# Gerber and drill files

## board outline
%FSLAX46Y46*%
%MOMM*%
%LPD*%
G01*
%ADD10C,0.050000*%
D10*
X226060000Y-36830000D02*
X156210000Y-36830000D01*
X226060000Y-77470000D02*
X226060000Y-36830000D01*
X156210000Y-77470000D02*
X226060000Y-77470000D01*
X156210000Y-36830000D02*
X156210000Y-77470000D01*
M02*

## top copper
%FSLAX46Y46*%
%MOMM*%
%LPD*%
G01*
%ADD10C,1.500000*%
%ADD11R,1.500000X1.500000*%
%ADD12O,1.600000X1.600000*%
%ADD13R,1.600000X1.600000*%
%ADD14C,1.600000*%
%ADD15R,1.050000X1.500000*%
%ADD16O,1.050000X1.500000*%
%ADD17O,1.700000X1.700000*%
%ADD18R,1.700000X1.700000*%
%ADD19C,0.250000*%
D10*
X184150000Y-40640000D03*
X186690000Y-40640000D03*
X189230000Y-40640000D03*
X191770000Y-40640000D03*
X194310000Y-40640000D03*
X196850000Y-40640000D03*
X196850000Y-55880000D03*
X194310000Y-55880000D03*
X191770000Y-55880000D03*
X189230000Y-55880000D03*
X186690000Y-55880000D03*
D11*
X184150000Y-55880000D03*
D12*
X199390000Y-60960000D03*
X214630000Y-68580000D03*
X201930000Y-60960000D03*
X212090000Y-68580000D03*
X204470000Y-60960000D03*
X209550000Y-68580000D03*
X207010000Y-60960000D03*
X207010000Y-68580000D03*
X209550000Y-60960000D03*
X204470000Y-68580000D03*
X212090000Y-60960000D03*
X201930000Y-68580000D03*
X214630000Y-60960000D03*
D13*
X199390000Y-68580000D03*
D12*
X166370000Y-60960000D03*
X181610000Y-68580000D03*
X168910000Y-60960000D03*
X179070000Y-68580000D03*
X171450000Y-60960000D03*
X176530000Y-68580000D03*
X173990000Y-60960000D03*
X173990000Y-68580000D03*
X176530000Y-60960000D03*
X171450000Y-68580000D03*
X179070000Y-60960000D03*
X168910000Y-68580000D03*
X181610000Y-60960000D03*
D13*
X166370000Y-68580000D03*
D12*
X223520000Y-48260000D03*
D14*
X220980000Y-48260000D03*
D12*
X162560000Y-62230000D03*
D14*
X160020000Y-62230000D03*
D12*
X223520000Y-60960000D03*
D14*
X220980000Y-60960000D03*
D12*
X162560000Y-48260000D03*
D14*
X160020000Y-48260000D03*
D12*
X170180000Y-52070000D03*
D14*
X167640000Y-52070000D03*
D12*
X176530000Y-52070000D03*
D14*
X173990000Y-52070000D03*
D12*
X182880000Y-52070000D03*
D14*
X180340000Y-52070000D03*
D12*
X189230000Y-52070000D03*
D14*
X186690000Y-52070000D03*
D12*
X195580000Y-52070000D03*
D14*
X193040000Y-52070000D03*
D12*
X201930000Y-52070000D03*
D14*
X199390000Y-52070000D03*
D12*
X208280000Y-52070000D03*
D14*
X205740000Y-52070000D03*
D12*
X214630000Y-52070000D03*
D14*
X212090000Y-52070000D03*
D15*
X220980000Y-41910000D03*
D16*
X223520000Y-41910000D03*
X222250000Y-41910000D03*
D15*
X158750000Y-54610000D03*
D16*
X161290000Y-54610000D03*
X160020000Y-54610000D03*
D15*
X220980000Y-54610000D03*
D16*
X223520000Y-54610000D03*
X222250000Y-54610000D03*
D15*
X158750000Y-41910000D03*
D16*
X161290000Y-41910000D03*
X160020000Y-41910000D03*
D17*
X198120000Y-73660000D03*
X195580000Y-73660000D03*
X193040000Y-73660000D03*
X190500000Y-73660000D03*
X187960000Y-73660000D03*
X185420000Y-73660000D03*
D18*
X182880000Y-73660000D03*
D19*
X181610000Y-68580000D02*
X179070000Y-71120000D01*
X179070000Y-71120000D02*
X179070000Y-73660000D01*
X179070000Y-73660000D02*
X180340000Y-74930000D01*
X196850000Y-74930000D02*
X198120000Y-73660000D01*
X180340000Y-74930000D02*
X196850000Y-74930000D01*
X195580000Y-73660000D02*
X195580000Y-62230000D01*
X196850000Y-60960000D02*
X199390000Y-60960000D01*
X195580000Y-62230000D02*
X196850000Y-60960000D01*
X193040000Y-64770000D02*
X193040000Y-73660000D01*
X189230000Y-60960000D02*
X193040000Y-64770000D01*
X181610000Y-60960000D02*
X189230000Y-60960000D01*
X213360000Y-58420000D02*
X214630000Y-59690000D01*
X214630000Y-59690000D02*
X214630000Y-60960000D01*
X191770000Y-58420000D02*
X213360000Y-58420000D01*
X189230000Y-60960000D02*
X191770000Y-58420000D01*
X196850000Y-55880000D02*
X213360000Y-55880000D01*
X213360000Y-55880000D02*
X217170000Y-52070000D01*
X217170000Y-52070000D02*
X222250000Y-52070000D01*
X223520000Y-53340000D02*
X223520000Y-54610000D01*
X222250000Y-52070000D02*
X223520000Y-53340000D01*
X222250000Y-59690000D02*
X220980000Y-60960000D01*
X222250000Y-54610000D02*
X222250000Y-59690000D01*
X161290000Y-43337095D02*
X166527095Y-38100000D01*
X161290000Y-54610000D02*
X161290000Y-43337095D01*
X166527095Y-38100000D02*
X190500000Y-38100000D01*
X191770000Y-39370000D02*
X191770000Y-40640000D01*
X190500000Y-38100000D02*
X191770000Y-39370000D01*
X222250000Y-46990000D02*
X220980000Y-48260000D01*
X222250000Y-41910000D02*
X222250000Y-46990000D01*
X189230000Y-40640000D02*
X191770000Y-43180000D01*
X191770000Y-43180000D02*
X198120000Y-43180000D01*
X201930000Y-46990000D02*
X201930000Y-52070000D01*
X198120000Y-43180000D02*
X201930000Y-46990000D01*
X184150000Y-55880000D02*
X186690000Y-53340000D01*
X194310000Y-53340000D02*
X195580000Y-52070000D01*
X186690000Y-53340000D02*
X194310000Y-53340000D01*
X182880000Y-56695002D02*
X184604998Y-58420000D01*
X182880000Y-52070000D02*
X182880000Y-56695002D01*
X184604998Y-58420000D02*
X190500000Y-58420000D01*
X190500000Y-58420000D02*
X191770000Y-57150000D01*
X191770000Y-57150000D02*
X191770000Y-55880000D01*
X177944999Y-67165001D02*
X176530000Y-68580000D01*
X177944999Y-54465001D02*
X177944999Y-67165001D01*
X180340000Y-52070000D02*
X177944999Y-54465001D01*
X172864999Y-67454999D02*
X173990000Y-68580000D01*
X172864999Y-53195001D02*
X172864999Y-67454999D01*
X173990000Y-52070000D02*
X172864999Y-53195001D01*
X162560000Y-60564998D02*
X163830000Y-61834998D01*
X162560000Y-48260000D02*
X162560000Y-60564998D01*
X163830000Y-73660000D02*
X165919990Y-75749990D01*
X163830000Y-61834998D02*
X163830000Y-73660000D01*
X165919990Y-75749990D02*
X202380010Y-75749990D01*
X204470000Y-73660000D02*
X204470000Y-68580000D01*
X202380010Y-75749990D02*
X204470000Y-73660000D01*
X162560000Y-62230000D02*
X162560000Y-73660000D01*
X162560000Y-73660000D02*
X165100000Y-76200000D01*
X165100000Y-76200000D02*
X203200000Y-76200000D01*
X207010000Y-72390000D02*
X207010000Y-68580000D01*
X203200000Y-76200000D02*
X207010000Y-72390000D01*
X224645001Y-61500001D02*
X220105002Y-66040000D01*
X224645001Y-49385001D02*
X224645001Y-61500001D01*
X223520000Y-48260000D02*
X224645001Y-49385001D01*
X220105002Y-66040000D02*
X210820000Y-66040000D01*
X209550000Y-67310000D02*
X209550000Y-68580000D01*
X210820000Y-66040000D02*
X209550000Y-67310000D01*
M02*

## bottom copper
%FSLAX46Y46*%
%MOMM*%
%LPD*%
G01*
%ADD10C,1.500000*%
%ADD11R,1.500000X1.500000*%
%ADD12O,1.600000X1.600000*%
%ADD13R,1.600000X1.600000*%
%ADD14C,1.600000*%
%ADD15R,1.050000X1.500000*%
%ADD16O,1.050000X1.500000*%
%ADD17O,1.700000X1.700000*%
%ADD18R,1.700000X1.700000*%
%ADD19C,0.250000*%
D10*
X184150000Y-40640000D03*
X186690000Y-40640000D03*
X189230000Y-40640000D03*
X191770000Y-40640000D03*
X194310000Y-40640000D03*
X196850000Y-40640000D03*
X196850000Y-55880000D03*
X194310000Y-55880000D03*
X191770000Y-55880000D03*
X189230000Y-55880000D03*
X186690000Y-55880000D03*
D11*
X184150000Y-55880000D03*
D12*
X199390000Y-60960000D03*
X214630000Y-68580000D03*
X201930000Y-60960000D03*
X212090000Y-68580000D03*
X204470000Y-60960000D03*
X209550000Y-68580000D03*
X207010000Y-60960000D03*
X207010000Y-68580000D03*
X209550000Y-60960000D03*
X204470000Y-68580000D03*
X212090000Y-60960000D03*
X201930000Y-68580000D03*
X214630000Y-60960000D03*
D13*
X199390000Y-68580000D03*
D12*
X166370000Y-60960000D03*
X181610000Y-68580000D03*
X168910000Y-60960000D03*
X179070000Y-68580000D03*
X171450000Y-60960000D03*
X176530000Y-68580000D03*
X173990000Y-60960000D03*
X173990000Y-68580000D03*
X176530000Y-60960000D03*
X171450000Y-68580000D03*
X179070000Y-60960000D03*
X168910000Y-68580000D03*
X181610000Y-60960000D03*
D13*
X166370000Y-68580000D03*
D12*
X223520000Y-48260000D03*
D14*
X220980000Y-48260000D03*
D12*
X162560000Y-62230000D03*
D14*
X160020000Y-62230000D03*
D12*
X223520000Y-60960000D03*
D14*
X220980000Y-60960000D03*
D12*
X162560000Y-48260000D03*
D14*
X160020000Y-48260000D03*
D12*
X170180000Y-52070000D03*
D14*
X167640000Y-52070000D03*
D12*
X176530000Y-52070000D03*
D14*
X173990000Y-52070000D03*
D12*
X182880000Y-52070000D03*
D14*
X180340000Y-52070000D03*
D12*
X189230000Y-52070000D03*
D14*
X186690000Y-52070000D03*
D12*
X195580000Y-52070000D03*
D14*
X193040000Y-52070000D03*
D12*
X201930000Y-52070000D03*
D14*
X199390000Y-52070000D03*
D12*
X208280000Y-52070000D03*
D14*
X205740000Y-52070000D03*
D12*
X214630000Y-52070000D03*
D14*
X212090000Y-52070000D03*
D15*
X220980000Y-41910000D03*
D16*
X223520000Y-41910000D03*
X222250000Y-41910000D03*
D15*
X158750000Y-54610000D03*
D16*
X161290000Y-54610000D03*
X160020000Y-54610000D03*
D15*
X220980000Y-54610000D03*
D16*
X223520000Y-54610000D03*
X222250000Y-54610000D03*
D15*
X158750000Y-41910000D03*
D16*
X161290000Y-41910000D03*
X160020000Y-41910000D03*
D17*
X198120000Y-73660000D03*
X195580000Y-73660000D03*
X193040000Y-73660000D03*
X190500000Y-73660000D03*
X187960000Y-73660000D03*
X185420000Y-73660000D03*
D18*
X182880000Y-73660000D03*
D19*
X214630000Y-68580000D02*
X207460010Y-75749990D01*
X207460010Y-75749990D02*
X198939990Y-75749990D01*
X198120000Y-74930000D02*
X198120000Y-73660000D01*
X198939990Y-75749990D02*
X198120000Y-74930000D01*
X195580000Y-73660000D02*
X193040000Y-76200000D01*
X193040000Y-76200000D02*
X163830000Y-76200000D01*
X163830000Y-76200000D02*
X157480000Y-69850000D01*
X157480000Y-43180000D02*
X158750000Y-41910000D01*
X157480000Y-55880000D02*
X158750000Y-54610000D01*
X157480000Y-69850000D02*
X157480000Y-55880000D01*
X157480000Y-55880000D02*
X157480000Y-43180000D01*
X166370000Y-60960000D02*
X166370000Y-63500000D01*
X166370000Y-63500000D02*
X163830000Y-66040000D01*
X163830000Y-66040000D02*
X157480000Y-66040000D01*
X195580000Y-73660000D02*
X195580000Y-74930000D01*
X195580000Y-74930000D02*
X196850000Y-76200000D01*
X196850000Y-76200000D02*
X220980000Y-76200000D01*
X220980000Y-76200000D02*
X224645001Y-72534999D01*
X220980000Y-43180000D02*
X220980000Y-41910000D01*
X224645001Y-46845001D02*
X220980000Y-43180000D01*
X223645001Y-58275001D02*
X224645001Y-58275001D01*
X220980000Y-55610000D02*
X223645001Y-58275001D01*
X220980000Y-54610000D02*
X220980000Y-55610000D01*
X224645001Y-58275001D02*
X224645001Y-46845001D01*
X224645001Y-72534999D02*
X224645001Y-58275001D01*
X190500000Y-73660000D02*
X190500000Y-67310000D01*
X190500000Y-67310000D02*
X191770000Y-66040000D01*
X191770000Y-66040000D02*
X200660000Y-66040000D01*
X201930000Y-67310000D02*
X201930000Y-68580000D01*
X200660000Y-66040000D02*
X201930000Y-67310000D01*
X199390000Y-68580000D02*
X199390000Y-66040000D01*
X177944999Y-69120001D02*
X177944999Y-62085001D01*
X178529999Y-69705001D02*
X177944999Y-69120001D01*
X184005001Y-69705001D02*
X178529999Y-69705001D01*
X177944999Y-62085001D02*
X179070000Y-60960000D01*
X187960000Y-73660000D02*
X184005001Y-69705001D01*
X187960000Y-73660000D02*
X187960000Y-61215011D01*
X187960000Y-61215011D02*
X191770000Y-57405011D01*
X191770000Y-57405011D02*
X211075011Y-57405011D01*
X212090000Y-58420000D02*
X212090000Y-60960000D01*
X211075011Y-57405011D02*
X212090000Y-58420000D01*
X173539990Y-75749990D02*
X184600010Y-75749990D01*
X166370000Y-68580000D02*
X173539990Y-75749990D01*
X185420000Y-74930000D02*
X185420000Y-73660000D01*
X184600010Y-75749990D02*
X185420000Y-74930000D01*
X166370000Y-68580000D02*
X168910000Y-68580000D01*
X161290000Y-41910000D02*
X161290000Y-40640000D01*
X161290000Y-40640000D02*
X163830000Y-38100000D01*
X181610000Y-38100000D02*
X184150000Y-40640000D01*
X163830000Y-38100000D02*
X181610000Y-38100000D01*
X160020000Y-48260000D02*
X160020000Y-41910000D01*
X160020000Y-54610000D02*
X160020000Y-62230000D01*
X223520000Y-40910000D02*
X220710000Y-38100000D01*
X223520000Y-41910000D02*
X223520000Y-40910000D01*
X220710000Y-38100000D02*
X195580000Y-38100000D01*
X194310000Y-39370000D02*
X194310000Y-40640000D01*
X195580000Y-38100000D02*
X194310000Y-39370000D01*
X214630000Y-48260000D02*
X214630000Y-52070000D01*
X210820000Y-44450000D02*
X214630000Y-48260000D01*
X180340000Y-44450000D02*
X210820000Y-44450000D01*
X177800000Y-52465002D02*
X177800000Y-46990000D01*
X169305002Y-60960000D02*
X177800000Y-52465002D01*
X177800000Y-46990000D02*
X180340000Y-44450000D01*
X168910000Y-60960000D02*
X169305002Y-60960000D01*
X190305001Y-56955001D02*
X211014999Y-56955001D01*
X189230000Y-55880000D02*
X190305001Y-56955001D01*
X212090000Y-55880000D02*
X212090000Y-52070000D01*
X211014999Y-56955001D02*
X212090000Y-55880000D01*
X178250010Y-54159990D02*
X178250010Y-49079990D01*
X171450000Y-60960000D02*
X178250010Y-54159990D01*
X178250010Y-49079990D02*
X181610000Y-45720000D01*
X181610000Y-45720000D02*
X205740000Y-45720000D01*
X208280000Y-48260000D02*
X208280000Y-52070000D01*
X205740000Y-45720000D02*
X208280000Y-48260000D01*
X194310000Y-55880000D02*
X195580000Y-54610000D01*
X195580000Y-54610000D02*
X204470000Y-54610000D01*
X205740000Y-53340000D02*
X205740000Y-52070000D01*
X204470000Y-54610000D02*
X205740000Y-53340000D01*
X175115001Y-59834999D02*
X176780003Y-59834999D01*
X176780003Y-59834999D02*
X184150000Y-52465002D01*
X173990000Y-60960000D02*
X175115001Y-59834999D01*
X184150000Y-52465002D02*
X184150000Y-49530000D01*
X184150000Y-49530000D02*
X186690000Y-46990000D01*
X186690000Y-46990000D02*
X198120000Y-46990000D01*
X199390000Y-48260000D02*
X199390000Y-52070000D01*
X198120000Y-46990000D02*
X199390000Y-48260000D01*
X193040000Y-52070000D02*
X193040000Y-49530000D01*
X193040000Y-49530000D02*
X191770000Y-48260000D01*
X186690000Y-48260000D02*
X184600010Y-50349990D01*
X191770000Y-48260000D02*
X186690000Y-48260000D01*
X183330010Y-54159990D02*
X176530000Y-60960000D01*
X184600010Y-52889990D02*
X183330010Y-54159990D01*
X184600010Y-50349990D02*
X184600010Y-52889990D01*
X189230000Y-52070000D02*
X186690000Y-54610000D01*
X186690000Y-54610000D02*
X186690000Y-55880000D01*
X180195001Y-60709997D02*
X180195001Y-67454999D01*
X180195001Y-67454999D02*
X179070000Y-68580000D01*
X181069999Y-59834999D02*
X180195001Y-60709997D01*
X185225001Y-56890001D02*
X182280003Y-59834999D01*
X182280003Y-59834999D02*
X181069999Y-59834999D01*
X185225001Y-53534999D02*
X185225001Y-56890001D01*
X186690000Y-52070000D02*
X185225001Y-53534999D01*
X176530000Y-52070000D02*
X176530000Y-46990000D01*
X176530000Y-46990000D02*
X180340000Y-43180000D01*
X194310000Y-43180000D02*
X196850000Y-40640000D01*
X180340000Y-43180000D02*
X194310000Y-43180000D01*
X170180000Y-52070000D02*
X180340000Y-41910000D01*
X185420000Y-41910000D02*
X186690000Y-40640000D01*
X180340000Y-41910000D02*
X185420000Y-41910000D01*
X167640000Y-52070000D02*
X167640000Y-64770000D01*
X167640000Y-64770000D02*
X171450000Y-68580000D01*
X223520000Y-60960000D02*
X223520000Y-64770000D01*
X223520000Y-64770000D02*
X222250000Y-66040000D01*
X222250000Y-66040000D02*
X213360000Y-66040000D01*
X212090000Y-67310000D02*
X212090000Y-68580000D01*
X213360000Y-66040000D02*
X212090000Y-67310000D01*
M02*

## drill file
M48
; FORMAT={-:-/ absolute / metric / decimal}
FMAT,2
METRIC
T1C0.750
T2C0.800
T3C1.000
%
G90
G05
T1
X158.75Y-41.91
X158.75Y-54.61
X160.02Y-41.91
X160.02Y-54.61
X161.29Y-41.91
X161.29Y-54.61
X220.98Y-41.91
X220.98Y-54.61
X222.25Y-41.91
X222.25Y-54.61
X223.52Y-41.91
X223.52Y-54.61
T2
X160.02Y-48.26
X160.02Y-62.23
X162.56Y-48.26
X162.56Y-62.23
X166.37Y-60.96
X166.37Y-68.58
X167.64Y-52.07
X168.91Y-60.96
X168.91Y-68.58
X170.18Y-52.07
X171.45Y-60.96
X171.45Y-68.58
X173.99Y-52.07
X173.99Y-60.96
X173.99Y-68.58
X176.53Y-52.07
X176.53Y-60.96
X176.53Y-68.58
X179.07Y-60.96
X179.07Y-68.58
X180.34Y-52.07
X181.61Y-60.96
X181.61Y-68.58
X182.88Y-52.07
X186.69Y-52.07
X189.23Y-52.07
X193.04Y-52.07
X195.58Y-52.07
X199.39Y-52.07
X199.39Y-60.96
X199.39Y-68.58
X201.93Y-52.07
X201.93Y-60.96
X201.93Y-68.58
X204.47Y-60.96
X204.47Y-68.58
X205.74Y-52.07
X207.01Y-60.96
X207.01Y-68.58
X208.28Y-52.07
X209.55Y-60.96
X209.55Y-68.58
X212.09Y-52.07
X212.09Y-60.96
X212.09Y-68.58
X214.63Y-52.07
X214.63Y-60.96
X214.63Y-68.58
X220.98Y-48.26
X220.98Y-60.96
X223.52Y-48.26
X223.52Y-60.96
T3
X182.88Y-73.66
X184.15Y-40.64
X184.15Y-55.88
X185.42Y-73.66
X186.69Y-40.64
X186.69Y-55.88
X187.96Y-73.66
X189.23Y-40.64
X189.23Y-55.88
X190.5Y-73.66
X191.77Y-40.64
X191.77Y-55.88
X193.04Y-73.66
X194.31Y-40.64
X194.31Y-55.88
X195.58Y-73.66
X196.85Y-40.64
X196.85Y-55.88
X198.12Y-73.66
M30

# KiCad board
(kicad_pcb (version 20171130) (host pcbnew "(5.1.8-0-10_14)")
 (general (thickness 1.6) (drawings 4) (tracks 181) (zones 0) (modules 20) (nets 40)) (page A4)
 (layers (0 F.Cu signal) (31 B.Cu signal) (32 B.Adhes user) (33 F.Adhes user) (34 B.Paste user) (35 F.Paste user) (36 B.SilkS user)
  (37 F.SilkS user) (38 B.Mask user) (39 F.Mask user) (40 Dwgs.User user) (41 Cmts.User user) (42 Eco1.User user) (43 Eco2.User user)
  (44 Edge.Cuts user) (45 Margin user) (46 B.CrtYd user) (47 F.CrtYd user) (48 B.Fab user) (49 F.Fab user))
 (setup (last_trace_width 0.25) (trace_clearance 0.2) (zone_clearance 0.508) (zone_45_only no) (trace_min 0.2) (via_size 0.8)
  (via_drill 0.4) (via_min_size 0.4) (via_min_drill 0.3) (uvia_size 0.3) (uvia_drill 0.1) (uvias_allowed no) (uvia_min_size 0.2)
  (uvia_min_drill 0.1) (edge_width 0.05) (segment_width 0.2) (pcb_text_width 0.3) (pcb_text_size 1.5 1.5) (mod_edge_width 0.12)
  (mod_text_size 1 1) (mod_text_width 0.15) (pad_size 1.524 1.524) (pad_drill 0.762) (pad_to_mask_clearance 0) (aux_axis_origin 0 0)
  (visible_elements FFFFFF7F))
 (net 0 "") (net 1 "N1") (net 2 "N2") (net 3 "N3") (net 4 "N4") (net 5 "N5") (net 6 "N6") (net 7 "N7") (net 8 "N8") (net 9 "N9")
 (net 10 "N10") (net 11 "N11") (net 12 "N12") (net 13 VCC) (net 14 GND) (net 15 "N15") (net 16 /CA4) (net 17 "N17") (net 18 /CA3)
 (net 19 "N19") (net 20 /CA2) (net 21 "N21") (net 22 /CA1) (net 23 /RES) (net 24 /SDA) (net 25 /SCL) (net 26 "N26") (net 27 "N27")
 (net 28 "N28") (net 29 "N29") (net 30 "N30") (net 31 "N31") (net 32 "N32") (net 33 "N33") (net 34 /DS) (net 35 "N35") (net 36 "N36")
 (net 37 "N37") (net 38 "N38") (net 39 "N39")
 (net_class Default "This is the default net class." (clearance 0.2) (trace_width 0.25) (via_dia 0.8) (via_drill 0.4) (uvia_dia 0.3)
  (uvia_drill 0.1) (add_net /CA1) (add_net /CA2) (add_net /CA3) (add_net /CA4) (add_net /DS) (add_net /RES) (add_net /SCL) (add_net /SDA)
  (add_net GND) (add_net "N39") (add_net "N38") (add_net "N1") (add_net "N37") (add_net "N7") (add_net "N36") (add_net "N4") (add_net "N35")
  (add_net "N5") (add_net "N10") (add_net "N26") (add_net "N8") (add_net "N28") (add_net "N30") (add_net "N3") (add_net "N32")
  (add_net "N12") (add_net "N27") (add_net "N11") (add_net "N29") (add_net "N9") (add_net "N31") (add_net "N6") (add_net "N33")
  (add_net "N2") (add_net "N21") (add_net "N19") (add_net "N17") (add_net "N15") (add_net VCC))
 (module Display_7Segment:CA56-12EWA (layer F.Cu) (at 184.15 55.88 90)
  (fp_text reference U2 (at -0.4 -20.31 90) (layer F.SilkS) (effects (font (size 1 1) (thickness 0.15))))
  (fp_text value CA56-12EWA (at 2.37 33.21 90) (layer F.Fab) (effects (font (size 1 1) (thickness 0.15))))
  (pad 12 thru_hole circle (at 15.24 0 90) (size 1.5 1.5) (drill 1) (layers *.Cu *.Mask) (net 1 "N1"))
  (pad 11 thru_hole circle (at 15.24 2.54 90) (size 1.5 1.5) (drill 1) (layers *.Cu *.Mask) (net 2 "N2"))
  (pad 10 thru_hole circle (at 15.24 5.08 90) (size 1.5 1.5) (drill 1) (layers *.Cu *.Mask) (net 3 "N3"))
  (pad 9 thru_hole circle (at 15.24 7.62 90) (size 1.5 1.5) (drill 1) (layers *.Cu *.Mask) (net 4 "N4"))
  (pad 8 thru_hole circle (at 15.24 10.16 90) (size 1.5 1.5) (drill 1) (layers *.Cu *.Mask) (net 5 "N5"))
  (pad 7 thru_hole circle (at 15.24 12.7 90) (size 1.5 1.5) (drill 1) (layers *.Cu *.Mask) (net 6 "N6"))
  (pad 6 thru_hole circle (at 0 12.7 90) (size 1.5 1.5) (drill 1) (layers *.Cu *.Mask) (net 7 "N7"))
  (pad 5 thru_hole circle (at 0 10.16 90) (size 1.5 1.5) (drill 1) (layers *.Cu *.Mask) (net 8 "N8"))
  (pad 4 thru_hole circle (at 0 7.62 90) (size 1.5 1.5) (drill 1) (layers *.Cu *.Mask) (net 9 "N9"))
  (pad 3 thru_hole circle (at 0 5.08 90) (size 1.5 1.5) (drill 1) (layers *.Cu *.Mask) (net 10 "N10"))
  (pad 2 thru_hole circle (at 0 2.54 90) (size 1.5 1.5) (drill 1) (layers *.Cu *.Mask) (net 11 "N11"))
  (pad 1 thru_hole rect (at 0 0 90) (size 1.5 1.5) (drill 1) (layers *.Cu *.Mask) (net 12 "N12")))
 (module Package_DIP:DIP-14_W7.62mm (layer F.Cu) (at 199.39 68.58 90)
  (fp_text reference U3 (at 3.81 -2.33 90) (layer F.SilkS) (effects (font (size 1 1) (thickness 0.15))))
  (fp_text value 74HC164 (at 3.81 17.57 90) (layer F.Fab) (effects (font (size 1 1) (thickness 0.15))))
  (pad 14 thru_hole oval (at 7.62 0 90) (size 1.6 1.6) (drill 0.8) (layers *.Cu *.Mask) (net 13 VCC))
  (pad 7 thru_hole oval (at 0 15.24 90) (size 1.6 1.6) (drill 0.8) (layers *.Cu *.Mask) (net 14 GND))
  (pad 13 thru_hole oval (at 7.62 2.54 90) (size 1.6 1.6) (drill 0.8) (layers *.Cu *.Mask) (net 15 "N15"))
  (pad 6 thru_hole oval (at 0 12.7 90) (size 1.6 1.6) (drill 0.8) (layers *.Cu *.Mask) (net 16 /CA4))
  (pad 12 thru_hole oval (at 7.62 5.08 90) (size 1.6 1.6) (drill 0.8) (layers *.Cu *.Mask) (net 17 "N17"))
  (pad 5 thru_hole oval (at 0 10.16 90) (size 1.6 1.6) (drill 0.8) (layers *.Cu *.Mask) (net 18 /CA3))
  (pad 11 thru_hole oval (at 7.62 7.62 90) (size 1.6 1.6) (drill 0.8) (layers *.Cu *.Mask) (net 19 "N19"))
  (pad 4 thru_hole oval (at 0 7.62 90) (size 1.6 1.6) (drill 0.8) (layers *.Cu *.Mask) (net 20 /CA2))
  (pad 10 thru_hole oval (at 7.62 10.16 90) (size 1.6 1.6) (drill 0.8) (layers *.Cu *.Mask) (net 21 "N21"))
  (pad 3 thru_hole oval (at 0 5.08 90) (size 1.6 1.6) (drill 0.8) (layers *.Cu *.Mask) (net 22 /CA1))
  (pad 9 thru_hole oval (at 7.62 12.7 90) (size 1.6 1.6) (drill 0.8) (layers *.Cu *.Mask) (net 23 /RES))
  (pad 2 thru_hole oval (at 0 2.54 90) (size 1.6 1.6) (drill 0.8) (layers *.Cu *.Mask) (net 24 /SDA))
  (pad 8 thru_hole oval (at 7.62 15.24 90) (size 1.6 1.6) (drill 0.8) (layers *.Cu *.Mask) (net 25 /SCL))
  (pad 1 thru_hole rect (at 0 0 90) (size 1.6 1.6) (drill 0.8) (layers *.Cu *.Mask) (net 24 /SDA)))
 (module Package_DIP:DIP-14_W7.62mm (layer F.Cu) (at 166.37 68.58 90)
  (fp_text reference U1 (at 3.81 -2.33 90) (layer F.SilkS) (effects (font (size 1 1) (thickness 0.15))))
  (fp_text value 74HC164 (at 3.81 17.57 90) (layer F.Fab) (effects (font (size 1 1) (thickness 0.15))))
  (pad 14 thru_hole oval (at 7.62 0 90) (size 1.6 1.6) (drill 0.8) (layers *.Cu *.Mask) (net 13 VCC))
  (pad 7 thru_hole oval (at 0 15.24 90) (size 1.6 1.6) (drill 0.8) (layers *.Cu *.Mask) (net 14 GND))
  (pad 13 thru_hole oval (at 7.62 2.54 90) (size 1.6 1.6) (drill 0.8) (layers *.Cu *.Mask) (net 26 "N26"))
  (pad 6 thru_hole oval (at 0 12.7 90) (size 1.6 1.6) (drill 0.8) (layers *.Cu *.Mask) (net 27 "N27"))
  (pad 12 thru_hole oval (at 7.62 5.08 90) (size 1.6 1.6) (drill 0.8) (layers *.Cu *.Mask) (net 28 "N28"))
  (pad 5 thru_hole oval (at 0 10.16 90) (size 1.6 1.6) (drill 0.8) (layers *.Cu *.Mask) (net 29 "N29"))
  (pad 11 thru_hole oval (at 7.62 7.62 90) (size 1.6 1.6) (drill 0.8) (layers *.Cu *.Mask) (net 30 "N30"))
  (pad 4 thru_hole oval (at 0 7.62 90) (size 1.6 1.6) (drill 0.8) (layers *.Cu *.Mask) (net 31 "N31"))
  (pad 10 thru_hole oval (at 7.62 10.16 90) (size 1.6 1.6) (drill 0.8) (layers *.Cu *.Mask) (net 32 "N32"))
  (pad 3 thru_hole oval (at 0 5.08 90) (size 1.6 1.6) (drill 0.8) (layers *.Cu *.Mask) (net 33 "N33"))
  (pad 9 thru_hole oval (at 7.62 12.7 90) (size 1.6 1.6) (drill 0.8) (layers *.Cu *.Mask) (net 23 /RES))
  (pad 2 thru_hole oval (at 0 2.54 90) (size 1.6 1.6) (drill 0.8) (layers *.Cu *.Mask) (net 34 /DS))
  (pad 8 thru_hole oval (at 7.62 15.24 90) (size 1.6 1.6) (drill 0.8) (layers *.Cu *.Mask) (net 25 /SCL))
  (pad 1 thru_hole rect (at 0 0 90) (size 1.6 1.6) (drill 0.8) (layers *.Cu *.Mask) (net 34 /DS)))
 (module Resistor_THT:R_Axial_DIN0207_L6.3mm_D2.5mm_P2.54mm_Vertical (layer F.Cu) (at 220.98 48.26)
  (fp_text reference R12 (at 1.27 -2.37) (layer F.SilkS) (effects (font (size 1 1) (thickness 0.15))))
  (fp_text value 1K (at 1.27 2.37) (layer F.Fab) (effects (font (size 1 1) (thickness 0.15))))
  (pad 2 thru_hole oval (at 2.54 0) (size 1.6 1.6) (drill 0.8) (layers *.Cu *.Mask) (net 18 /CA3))
  (pad 1 thru_hole circle (at 0 0) (size 1.6 1.6) (drill 0.8) (layers *.Cu *.Mask) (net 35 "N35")))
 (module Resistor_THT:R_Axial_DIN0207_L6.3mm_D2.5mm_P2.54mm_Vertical (layer F.Cu) (at 160.02 62.23)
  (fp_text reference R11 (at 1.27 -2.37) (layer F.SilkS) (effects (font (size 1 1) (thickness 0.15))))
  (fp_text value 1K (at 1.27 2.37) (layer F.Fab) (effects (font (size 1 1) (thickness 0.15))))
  (pad 2 thru_hole oval (at 2.54 0) (size 1.6 1.6) (drill 0.8) (layers *.Cu *.Mask) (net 20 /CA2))
  (pad 1 thru_hole circle (at 0 0) (size 1.6 1.6) (drill 0.8) (layers *.Cu *.Mask) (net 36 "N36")))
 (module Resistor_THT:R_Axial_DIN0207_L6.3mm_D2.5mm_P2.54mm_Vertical (layer F.Cu) (at 220.98 60.96)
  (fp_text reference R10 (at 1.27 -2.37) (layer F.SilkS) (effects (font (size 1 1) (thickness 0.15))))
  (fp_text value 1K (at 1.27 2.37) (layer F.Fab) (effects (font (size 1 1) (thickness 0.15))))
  (pad 2 thru_hole oval (at 2.54 0) (size 1.6 1.6) (drill 0.8) (layers *.Cu *.Mask) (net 16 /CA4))
  (pad 1 thru_hole circle (at 0 0) (size 1.6 1.6) (drill 0.8) (layers *.Cu *.Mask) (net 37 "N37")))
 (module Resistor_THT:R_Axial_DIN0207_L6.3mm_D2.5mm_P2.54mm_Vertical (layer F.Cu) (at 160.02 48.26)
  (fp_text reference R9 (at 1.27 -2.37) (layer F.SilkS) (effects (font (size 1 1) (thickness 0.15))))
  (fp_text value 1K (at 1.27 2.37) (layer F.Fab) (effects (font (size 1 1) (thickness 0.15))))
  (pad 2 thru_hole oval (at 2.54 0) (size 1.6 1.6) (drill 0.8) (layers *.Cu *.Mask) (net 22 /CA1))
  (pad 1 thru_hole circle (at 0 0) (size 1.6 1.6) (drill 0.8) (layers *.Cu *.Mask) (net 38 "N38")))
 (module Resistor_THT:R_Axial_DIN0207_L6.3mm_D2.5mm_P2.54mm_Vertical (layer B.Cu) (at 167.64 52.07)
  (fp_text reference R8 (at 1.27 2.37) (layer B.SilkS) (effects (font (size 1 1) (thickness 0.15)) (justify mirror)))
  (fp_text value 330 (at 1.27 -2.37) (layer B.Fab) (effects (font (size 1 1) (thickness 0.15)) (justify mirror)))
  (pad 2 thru_hole oval (at 2.54 0) (size 1.6 1.6) (drill 0.8) (layers *.Cu *.Mask) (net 2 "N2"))
  (pad 1 thru_hole circle (at 0 0) (size 1.6 1.6) (drill 0.8) (layers *.Cu *.Mask) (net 33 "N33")))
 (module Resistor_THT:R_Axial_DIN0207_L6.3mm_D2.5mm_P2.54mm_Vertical (layer B.Cu) (at 173.99 52.07)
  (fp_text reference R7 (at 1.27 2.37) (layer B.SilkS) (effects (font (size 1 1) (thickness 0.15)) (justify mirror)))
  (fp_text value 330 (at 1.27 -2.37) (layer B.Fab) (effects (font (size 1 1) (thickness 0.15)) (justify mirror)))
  (pad 2 thru_hole oval (at 2.54 0) (size 1.6 1.6) (drill 0.8) (layers *.Cu *.Mask) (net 6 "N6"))
  (pad 1 thru_hole circle (at 0 0) (size 1.6 1.6) (drill 0.8) (layers *.Cu *.Mask) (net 31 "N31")))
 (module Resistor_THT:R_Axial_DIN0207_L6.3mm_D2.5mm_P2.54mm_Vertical (layer B.Cu) (at 180.34 52.07)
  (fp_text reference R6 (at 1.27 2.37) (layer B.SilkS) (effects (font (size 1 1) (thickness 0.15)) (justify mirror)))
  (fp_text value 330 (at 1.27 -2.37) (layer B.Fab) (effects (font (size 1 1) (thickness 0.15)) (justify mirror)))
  (pad 2 thru_hole oval (at 2.54 0) (size 1.6 1.6) (drill 0.8) (layers *.Cu *.Mask) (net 9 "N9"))
  (pad 1 thru_hole circle (at 0 0) (size 1.6 1.6) (drill 0.8) (layers *.Cu *.Mask) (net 29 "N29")))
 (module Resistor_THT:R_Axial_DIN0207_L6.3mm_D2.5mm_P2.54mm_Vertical (layer B.Cu) (at 186.69 52.07)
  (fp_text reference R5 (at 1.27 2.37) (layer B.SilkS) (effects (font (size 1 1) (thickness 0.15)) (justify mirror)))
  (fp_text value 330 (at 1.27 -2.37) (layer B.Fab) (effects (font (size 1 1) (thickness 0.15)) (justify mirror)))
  (pad 2 thru_hole oval (at 2.54 0) (size 1.6 1.6) (drill 0.8) (layers *.Cu *.Mask) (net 11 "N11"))
  (pad 1 thru_hole circle (at 0 0) (size 1.6 1.6) (drill 0.8) (layers *.Cu *.Mask) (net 27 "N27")))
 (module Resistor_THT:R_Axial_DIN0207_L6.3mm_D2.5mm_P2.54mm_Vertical (layer B.Cu) (at 193.04 52.07)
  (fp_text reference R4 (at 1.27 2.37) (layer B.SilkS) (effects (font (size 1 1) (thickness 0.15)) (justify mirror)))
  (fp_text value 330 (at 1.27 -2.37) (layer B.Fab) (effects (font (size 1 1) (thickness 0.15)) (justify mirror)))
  (pad 2 thru_hole oval (at 2.54 0) (size 1.6 1.6) (drill 0.8) (layers *.Cu *.Mask) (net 12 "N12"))
  (pad 1 thru_hole circle (at 0 0) (size 1.6 1.6) (drill 0.8) (layers *.Cu *.Mask) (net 32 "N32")))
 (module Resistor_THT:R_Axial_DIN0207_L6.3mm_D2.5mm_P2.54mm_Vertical (layer B.Cu) (at 199.39 52.07)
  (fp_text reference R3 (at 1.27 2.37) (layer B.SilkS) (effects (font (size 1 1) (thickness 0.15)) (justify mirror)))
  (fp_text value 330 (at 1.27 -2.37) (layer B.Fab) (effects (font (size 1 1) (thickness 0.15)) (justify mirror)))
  (pad 2 thru_hole oval (at 2.54 0) (size 1.6 1.6) (drill 0.8) (layers *.Cu *.Mask) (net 3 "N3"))
  (pad 1 thru_hole circle (at 0 0) (size 1.6 1.6) (drill 0.8) (layers *.Cu *.Mask) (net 30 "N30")))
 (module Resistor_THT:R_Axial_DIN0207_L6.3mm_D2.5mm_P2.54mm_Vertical (layer B.Cu) (at 205.74 52.07)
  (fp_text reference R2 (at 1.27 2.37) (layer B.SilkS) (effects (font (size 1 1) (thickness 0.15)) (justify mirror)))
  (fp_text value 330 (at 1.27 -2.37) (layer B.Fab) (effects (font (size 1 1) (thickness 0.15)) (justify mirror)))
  (pad 2 thru_hole oval (at 2.54 0) (size 1.6 1.6) (drill 0.8) (layers *.Cu *.Mask) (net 28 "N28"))
  (pad 1 thru_hole circle (at 0 0) (size 1.6 1.6) (drill 0.8) (layers *.Cu *.Mask) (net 8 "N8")))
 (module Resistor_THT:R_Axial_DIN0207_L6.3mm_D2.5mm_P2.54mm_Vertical (layer B.Cu) (at 212.09 52.07)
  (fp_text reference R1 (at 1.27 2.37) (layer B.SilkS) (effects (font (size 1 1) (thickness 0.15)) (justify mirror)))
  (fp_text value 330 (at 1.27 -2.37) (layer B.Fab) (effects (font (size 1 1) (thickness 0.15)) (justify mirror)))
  (pad 2 thru_hole oval (at 2.54 0) (size 1.6 1.6) (drill 0.8) (layers *.Cu *.Mask) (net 26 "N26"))
  (pad 1 thru_hole circle (at 0 0) (size 1.6 1.6) (drill 0.8) (layers *.Cu *.Mask) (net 10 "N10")))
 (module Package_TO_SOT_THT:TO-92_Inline (layer F.Cu) (at 220.98 41.91)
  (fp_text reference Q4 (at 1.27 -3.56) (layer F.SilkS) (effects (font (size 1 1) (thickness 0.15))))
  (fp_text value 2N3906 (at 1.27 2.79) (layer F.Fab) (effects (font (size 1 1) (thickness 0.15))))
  (pad 1 thru_hole rect (at 0 0) (size 1.05 1.5) (drill 0.75) (layers *.Cu *.Mask) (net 13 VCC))
  (pad 3 thru_hole oval (at 2.54 0) (size 1.05 1.5) (drill 0.75) (layers *.Cu *.Mask) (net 5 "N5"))
  (pad 2 thru_hole oval (at 1.27 0) (size 1.05 1.5) (drill 0.75) (layers *.Cu *.Mask) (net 35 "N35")))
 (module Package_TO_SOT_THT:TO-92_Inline (layer F.Cu) (at 158.75 54.61)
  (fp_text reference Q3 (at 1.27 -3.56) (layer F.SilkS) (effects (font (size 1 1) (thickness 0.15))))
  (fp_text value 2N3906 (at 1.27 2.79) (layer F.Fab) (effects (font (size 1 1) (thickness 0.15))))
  (pad 1 thru_hole rect (at 0 0) (size 1.05 1.5) (drill 0.75) (layers *.Cu *.Mask) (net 13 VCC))
  (pad 3 thru_hole oval (at 2.54 0) (size 1.05 1.5) (drill 0.75) (layers *.Cu *.Mask) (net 4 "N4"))
  (pad 2 thru_hole oval (at 1.27 0) (size 1.05 1.5) (drill 0.75) (layers *.Cu *.Mask) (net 36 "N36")))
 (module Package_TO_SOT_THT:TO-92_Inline (layer F.Cu) (at 220.98 54.61)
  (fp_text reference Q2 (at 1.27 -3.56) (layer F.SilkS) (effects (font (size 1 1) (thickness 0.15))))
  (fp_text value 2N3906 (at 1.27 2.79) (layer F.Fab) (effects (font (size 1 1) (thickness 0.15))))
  (pad 1 thru_hole rect (at 0 0) (size 1.05 1.5) (drill 0.75) (layers *.Cu *.Mask) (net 13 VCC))
  (pad 3 thru_hole oval (at 2.54 0) (size 1.05 1.5) (drill 0.75) (layers *.Cu *.Mask) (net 7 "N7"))
  (pad 2 thru_hole oval (at 1.27 0) (size 1.05 1.5) (drill 0.75) (layers *.Cu *.Mask) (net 37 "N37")))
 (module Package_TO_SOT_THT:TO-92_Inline (layer F.Cu) (at 158.75 41.91)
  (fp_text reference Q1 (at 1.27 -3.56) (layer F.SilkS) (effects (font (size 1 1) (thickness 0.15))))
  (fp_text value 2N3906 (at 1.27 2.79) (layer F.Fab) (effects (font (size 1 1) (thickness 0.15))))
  (pad 1 thru_hole rect (at 0 0) (size 1.05 1.5) (drill 0.75) (layers *.Cu *.Mask) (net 13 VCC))
  (pad 3 thru_hole oval (at 2.54 0) (size 1.05 1.5) (drill 0.75) (layers *.Cu *.Mask) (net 1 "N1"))
  (pad 2 thru_hole oval (at 1.27 0) (size 1.05 1.5) (drill 0.75) (layers *.Cu *.Mask) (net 38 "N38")))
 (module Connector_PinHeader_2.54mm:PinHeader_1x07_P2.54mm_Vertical (layer B.Cu) (at 182.88 73.66 270)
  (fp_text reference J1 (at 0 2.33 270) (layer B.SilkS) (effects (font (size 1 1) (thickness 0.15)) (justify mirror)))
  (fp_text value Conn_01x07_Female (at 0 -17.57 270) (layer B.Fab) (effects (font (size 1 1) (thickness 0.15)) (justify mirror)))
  (pad 7 thru_hole oval (at 0 -15.24 270) (size 1.7 1.7) (drill 1) (layers *.Cu *.Mask) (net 14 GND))
  (pad 6 thru_hole oval (at 0 -12.7 270) (size 1.7 1.7) (drill 1) (layers *.Cu *.Mask) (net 13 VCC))
  (pad 5 thru_hole oval (at 0 -10.16 270) (size 1.7 1.7) (drill 1) (layers *.Cu *.Mask) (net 25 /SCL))
  (pad 4 thru_hole oval (at 0 -7.62 270) (size 1.7 1.7) (drill 1) (layers *.Cu *.Mask) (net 24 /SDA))
  (pad 3 thru_hole oval (at 0 -5.08 270) (size 1.7 1.7) (drill 1) (layers *.Cu *.Mask) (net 23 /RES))
  (pad 2 thru_hole oval (at 0 -2.54 270) (size 1.7 1.7) (drill 1) (layers *.Cu *.Mask) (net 34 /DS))
  (pad 1 thru_hole rect (at 0 0 270) (size 1.7 1.7) (drill 1) (layers *.Cu *.Mask) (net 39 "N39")))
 (gr_line (start 226.06 36.83) (end 156.21 36.83) (layer Edge.Cuts) (width 0.05))
 (gr_line (start 226.06 77.47) (end 226.06 36.83) (layer Edge.Cuts) (width 0.05))
 (gr_line (start 156.21 77.47) (end 226.06 77.47) (layer Edge.Cuts) (width 0.05))
 (gr_line (start 156.21 36.83) (end 156.21 77.47) (layer Edge.Cuts) (width 0.05))
 (segment (start 181.61 68.58) (end 179.07 71.12) (width 0.25) (layer F.Cu) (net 14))
 (segment (start 179.07 71.12) (end 179.07 73.66) (width 0.25) (layer F.Cu) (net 14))
 (segment (start 179.07 73.66) (end 180.34 74.93) (width 0.25) (layer F.Cu) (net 14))
 (segment (start 196.85 74.93) (end 198.12 73.66) (width 0.25) (layer F.Cu) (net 14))
 (segment (start 180.34 74.93) (end 196.85 74.93) (width 0.25) (layer F.Cu) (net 14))
 (segment (start 214.63 68.58) (end 207.46001 75.74999) (width 0.25) (layer B.Cu) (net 14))
 (segment (start 207.46001 75.74999) (end 198.93999 75.74999) (width 0.25) (layer B.Cu) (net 14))
 (segment (start 198.12 74.93) (end 198.12 73.66) (width 0.25) (layer B.Cu) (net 14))
 (segment (start 198.93999 75.74999) (end 198.12 74.93) (width 0.25) (layer B.Cu) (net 14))
 (segment (start 195.58 73.66) (end 193.04 76.2) (width 0.25) (layer B.Cu) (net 13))
 (segment (start 193.04 76.2) (end 163.83 76.2) (width 0.25) (layer B.Cu) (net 13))
 (segment (start 163.83 76.2) (end 157.48 69.85) (width 0.25) (layer B.Cu) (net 13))
 (segment (start 157.48 43.18) (end 158.75 41.91) (width 0.25) (layer B.Cu) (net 13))
 (segment (start 157.48 55.88) (end 158.75 54.61) (width 0.25) (layer B.Cu) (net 13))
 (segment (start 157.48 69.85) (end 157.48 55.88) (width 0.25) (layer B.Cu) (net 13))
 (segment (start 157.48 55.88) (end 157.48 43.18) (width 0.25) (layer B.Cu) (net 13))
 (segment (start 166.37 60.96) (end 166.37 63.5) (width 0.25) (layer B.Cu) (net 13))
 (segment (start 166.37 63.5) (end 163.83 66.04) (width 0.25) (layer B.Cu) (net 13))
 (segment (start 163.83 66.04) (end 157.48 66.04) (width 0.25) (layer B.Cu) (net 13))
 (segment (start 195.58 73.66) (end 195.58 74.93) (width 0.25) (layer B.Cu) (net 13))
 (segment (start 195.58 74.93) (end 196.85 76.2) (width 0.25) (layer B.Cu) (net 13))
 (segment (start 196.85 76.2) (end 220.98 76.2) (width 0.25) (layer B.Cu) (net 13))
 (segment (start 220.98 76.2) (end 224.645001 72.534999) (width 0.25) (layer B.Cu) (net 13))
 (segment (start 220.98 43.18) (end 220.98 41.91) (width 0.25) (layer B.Cu) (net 13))
 (segment (start 224.645001 46.845001) (end 220.98 43.18) (width 0.25) (layer B.Cu) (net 13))
 (segment (start 223.645001 58.275001) (end 224.645001 58.275001) (width 0.25) (layer B.Cu) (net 13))
 (segment (start 220.98 55.61) (end 223.645001 58.275001) (width 0.25) (layer B.Cu) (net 13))
 (segment (start 220.98 54.61) (end 220.98 55.61) (width 0.25) (layer B.Cu) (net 13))
 (segment (start 224.645001 58.275001) (end 224.645001 46.845001) (width 0.25) (layer B.Cu) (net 13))
 (segment (start 224.645001 72.534999) (end 224.645001 58.275001) (width 0.25) (layer B.Cu) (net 13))
 (segment (start 195.58 73.66) (end 195.58 62.23) (width 0.25) (layer F.Cu) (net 13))
 (segment (start 196.85 60.96) (end 199.39 60.96) (width 0.25) (layer F.Cu) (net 13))
 (segment (start 195.58 62.23) (end 196.85 60.96) (width 0.25) (layer F.Cu) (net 13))
 (segment (start 193.04 64.77) (end 193.04 73.66) (width 0.25) (layer F.Cu) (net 25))
 (segment (start 189.23 60.96) (end 193.04 64.77) (width 0.25) (layer F.Cu) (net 25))
 (segment (start 181.61 60.96) (end 189.23 60.96) (width 0.25) (layer F.Cu) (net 25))
 (segment (start 213.36 58.42) (end 214.63 59.69) (width 0.25) (layer F.Cu) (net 25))
 (segment (start 214.63 59.69) (end 214.63 60.96) (width 0.25) (layer F.Cu) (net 25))
 (segment (start 191.77 58.42) (end 213.36 58.42) (width 0.25) (layer F.Cu) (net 25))
 (segment (start 189.23 60.96) (end 191.77 58.42) (width 0.25) (layer F.Cu) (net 25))
 (segment (start 190.5 73.66) (end 190.5 67.31) (width 0.25) (layer B.Cu) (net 24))
 (segment (start 190.5 67.31) (end 191.77 66.04) (width 0.25) (layer B.Cu) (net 24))
 (segment (start 191.77 66.04) (end 200.66 66.04) (width 0.25) (layer B.Cu) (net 24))
 (segment (start 201.93 67.31) (end 201.93 68.58) (width 0.25) (layer B.Cu) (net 24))
 (segment (start 200.66 66.04) (end 201.93 67.31) (width 0.25) (layer B.Cu) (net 24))
 (segment (start 199.39 68.58) (end 199.39 66.04) (width 0.25) (layer B.Cu) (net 24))
 (segment (start 177.944999 69.120001) (end 177.944999 62.085001) (width 0.25) (layer B.Cu) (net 23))
 (segment (start 178.529999 69.705001) (end 177.944999 69.120001) (width 0.25) (layer B.Cu) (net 23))
 (segment (start 184.005001 69.705001) (end 178.529999 69.705001) (width 0.25) (layer B.Cu) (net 23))
 (segment (start 177.944999 62.085001) (end 179.07 60.96) (width 0.25) (layer B.Cu) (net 23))
 (segment (start 187.96 73.66) (end 184.005001 69.705001) (width 0.25) (layer B.Cu) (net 23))
 (segment (start 187.96 73.66) (end 187.96 61.215011) (width 0.25) (layer B.Cu) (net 23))
 (segment (start 187.96 61.215011) (end 191.77 57.405011) (width 0.25) (layer B.Cu) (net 23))
 (segment (start 191.77 57.405011) (end 211.075011 57.405011) (width 0.25) (layer B.Cu) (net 23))
 (segment (start 212.09 58.42) (end 212.09 60.96) (width 0.25) (layer B.Cu) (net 23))
 (segment (start 211.075011 57.405011) (end 212.09 58.42) (width 0.25) (layer B.Cu) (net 23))
 (segment (start 173.53999 75.74999) (end 184.60001 75.74999) (width 0.25) (layer B.Cu) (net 34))
 (segment (start 166.37 68.58) (end 173.53999 75.74999) (width 0.25) (layer B.Cu) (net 34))
 (segment (start 185.42 74.93) (end 185.42 73.66) (width 0.25) (layer B.Cu) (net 34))
 (segment (start 184.60001 75.74999) (end 185.42 74.93) (width 0.25) (layer B.Cu) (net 34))
 (segment (start 166.37 68.58) (end 168.91 68.58) (width 0.25) (layer B.Cu) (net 34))
 (segment (start 161.29 41.91) (end 161.29 40.64) (width 0.25) (layer B.Cu) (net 1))
 (segment (start 161.29 40.64) (end 163.83 38.1) (width 0.25) (layer B.Cu) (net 1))
 (segment (start 181.61 38.1) (end 184.15 40.64) (width 0.25) (layer B.Cu) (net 1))
 (segment (start 163.83 38.1) (end 181.61 38.1) (width 0.25) (layer B.Cu) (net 1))
 (segment (start 160.02 48.26) (end 160.02 41.91) (width 0.25) (layer B.Cu) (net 38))
 (segment (start 196.85 55.88) (end 213.36 55.88) (width 0.25) (layer F.Cu) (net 7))
 (segment (start 213.36 55.88) (end 217.17 52.07) (width 0.25) (layer F.Cu) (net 7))
 (segment (start 217.17 52.07) (end 222.25 52.07) (width 0.25) (layer F.Cu) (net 7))
 (segment (start 223.52 53.34) (end 223.52 54.61) (width 0.25) (layer F.Cu) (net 7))
 (segment (start 222.25 52.07) (end 223.52 53.34) (width 0.25) (layer F.Cu) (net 7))
 (segment (start 222.25 59.69) (end 220.98 60.96) (width 0.25) (layer F.Cu) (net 37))
 (segment (start 222.25 54.61) (end 222.25 59.69) (width 0.25) (layer F.Cu) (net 37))
 (segment (start 161.29 43.337095) (end 166.527095 38.1) (width 0.25) (layer F.Cu) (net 4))
 (segment (start 161.29 54.61) (end 161.29 43.337095) (width 0.25) (layer F.Cu) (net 4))
 (segment (start 166.527095 38.1) (end 190.5 38.1) (width 0.25) (layer F.Cu) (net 4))
 (segment (start 191.77 39.37) (end 191.77 40.64) (width 0.25) (layer F.Cu) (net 4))
 (segment (start 190.5 38.1) (end 191.77 39.37) (width 0.25) (layer F.Cu) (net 4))
 (segment (start 160.02 54.61) (end 160.02 62.23) (width 0.25) (layer B.Cu) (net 36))
 (segment (start 223.52 40.91) (end 220.71 38.1) (width 0.25) (layer B.Cu) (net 5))
 (segment (start 223.52 41.91) (end 223.52 40.91) (width 0.25) (layer B.Cu) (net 5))
 (segment (start 220.71 38.1) (end 195.58 38.1) (width 0.25) (layer B.Cu) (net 5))
 (segment (start 194.31 39.37) (end 194.31 40.64) (width 0.25) (layer B.Cu) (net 5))
 (segment (start 195.58 38.1) (end 194.31 39.37) (width 0.25) (layer B.Cu) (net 5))
 (segment (start 222.25 46.99) (end 220.98 48.26) (width 0.25) (layer F.Cu) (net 35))
 (segment (start 222.25 41.91) (end 222.25 46.99) (width 0.25) (layer F.Cu) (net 35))
 (segment (start 214.63 48.26) (end 214.63 52.07) (width 0.25) (layer B.Cu) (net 26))
 (segment (start 210.82 44.45) (end 214.63 48.26) (width 0.25) (layer B.Cu) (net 26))
 (segment (start 180.34 44.45) (end 210.82 44.45) (width 0.25) (layer B.Cu) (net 26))
 (segment (start 177.8 52.465002) (end 177.8 46.99) (width 0.25) (layer B.Cu) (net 26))
 (segment (start 169.305002 60.96) (end 177.8 52.465002) (width 0.25) (layer B.Cu) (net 26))
 (segment (start 177.8 46.99) (end 180.34 44.45) (width 0.25) (layer B.Cu) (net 26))
 (segment (start 168.91 60.96) (end 169.305002 60.96) (width 0.25) (layer B.Cu) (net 26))
 (segment (start 190.305001 56.955001) (end 211.014999 56.955001) (width 0.25) (layer B.Cu) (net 10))
 (segment (start 189.23 55.88) (end 190.305001 56.955001) (width 0.25) (layer B.Cu) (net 10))
 (segment (start 212.09 55.88) (end 212.09 52.07) (width 0.25) (layer B.Cu) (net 10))
 (segment (start 211.014999 56.955001) (end 212.09 55.88) (width 0.25) (layer B.Cu) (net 10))
 (segment (start 178.25001 54.15999) (end 178.25001 49.07999) (width 0.25) (layer B.Cu) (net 28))
 (segment (start 171.45 60.96) (end 178.25001 54.15999) (width 0.25) (layer B.Cu) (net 28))
 (segment (start 178.25001 49.07999) (end 181.61 45.72) (width 0.25) (layer B.Cu) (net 28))
 (segment (start 181.61 45.72) (end 205.74 45.72) (width 0.25) (layer B.Cu) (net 28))
 (segment (start 208.28 48.26) (end 208.28 52.07) (width 0.25) (layer B.Cu) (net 28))
 (segment (start 205.74 45.72) (end 208.28 48.26) (width 0.25) (layer B.Cu) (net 28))
 (segment (start 194.31 55.88) (end 195.58 54.61) (width 0.25) (layer B.Cu) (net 8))
 (segment (start 195.58 54.61) (end 204.47 54.61) (width 0.25) (layer B.Cu) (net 8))
 (segment (start 205.74 53.34) (end 205.74 52.07) (width 0.25) (layer B.Cu) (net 8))
 (segment (start 204.47 54.61) (end 205.74 53.34) (width 0.25) (layer B.Cu) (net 8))
 (segment (start 189.23 40.64) (end 191.77 43.18) (width 0.25) (layer F.Cu) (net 3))
 (segment (start 191.77 43.18) (end 198.12 43.18) (width 0.25) (layer F.Cu) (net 3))
 (segment (start 201.93 46.99) (end 201.93 52.07) (width 0.25) (layer F.Cu) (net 3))
 (segment (start 198.12 43.18) (end 201.93 46.99) (width 0.25) (layer F.Cu) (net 3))
 (segment (start 175.115001 59.834999) (end 176.780003 59.834999) (width 0.25) (layer B.Cu) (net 30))
 (segment (start 176.780003 59.834999) (end 184.15 52.465002) (width 0.25) (layer B.Cu) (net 30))
 (segment (start 173.99 60.96) (end 175.115001 59.834999) (width 0.25) (layer B.Cu) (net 30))
 (segment (start 184.15 52.465002) (end 184.15 49.53) (width 0.25) (layer B.Cu) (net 30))
 (segment (start 184.15 49.53) (end 186.69 46.99) (width 0.25) (layer B.Cu) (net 30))
 (segment (start 186.69 46.99) (end 198.12 46.99) (width 0.25) (layer B.Cu) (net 30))
 (segment (start 199.39 48.26) (end 199.39 52.07) (width 0.25) (layer B.Cu) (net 30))
 (segment (start 198.12 46.99) (end 199.39 48.26) (width 0.25) (layer B.Cu) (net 30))
 (segment (start 184.15 55.88) (end 186.69 53.34) (width 0.25) (layer F.Cu) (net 12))
 (segment (start 194.31 53.34) (end 195.58 52.07) (width 0.25) (layer F.Cu) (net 12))
 (segment (start 186.69 53.34) (end 194.31 53.34) (width 0.25) (layer F.Cu) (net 12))
 (segment (start 193.04 52.07) (end 193.04 49.53) (width 0.25) (layer B.Cu) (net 32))
 (segment (start 193.04 49.53) (end 191.77 48.26) (width 0.25) (layer B.Cu) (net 32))
 (segment (start 186.69 48.26) (end 184.60001 50.34999) (width 0.25) (layer B.Cu) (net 32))
 (segment (start 191.77 48.26) (end 186.69 48.26) (width 0.25) (layer B.Cu) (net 32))
 (segment (start 183.33001 54.15999) (end 176.53 60.96) (width 0.25) (layer B.Cu) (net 32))
 (segment (start 184.60001 52.88999) (end 183.33001 54.15999) (width 0.25) (layer B.Cu) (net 32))
 (segment (start 184.60001 50.34999) (end 184.60001 52.88999) (width 0.25) (layer B.Cu) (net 32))
 (segment (start 189.23 52.07) (end 186.69 54.61) (width 0.25) (layer B.Cu) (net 11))
 (segment (start 186.69 54.61) (end 186.69 55.88) (width 0.25) (layer B.Cu) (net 11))
 (segment (start 180.195001 60.709997) (end 180.195001 67.454999) (width 0.25) (layer B.Cu) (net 27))
 (segment (start 180.195001 67.454999) (end 179.07 68.58) (width 0.25) (layer B.Cu) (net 27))
 (segment (start 181.069999 59.834999) (end 180.195001 60.709997) (width 0.25) (layer B.Cu) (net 27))
 (segment (start 185.225001 56.890001) (end 182.280003 59.834999) (width 0.25) (layer B.Cu) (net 27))
 (segment (start 182.280003 59.834999) (end 181.069999 59.834999) (width 0.25) (layer B.Cu) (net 27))
 (segment (start 185.225001 53.534999) (end 185.225001 56.890001) (width 0.25) (layer B.Cu) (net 27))
 (segment (start 186.69 52.07) (end 185.225001 53.534999) (width 0.25) (layer B.Cu) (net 27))
 (segment (start 182.88 56.695002) (end 184.604998 58.42) (width 0.25) (layer F.Cu) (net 9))
 (segment (start 182.88 52.07) (end 182.88 56.695002) (width 0.25) (layer F.Cu) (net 9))
 (segment (start 184.604998 58.42) (end 190.5 58.42) (width 0.25) (layer F.Cu) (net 9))
 (segment (start 190.5 58.42) (end 191.77 57.15) (width 0.25) (layer F.Cu) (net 9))
 (segment (start 191.77 57.15) (end 191.77 55.88) (width 0.25) (layer F.Cu) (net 9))
 (segment (start 177.944999 67.165001) (end 176.53 68.58) (width 0.25) (layer F.Cu) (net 29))
 (segment (start 177.944999 54.465001) (end 177.944999 67.165001) (width 0.25) (layer F.Cu) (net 29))
 (segment (start 180.34 52.07) (end 177.944999 54.465001) (width 0.25) (layer F.Cu) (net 29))
 (segment (start 176.53 52.07) (end 176.53 46.99) (width 0.25) (layer B.Cu) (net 6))
 (segment (start 176.53 46.99) (end 180.34 43.18) (width 0.25) (layer B.Cu) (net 6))
 (segment (start 194.31 43.18) (end 196.85 40.64) (width 0.25) (layer B.Cu) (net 6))
 (segment (start 180.34 43.18) (end 194.31 43.18) (width 0.25) (layer B.Cu) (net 6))
 (segment (start 172.864999 67.454999) (end 173.99 68.58) (width 0.25) (layer F.Cu) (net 31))
 (segment (start 172.864999 53.195001) (end 172.864999 67.454999) (width 0.25) (layer F.Cu) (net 31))
 (segment (start 173.99 52.07) (end 172.864999 53.195001) (width 0.25) (layer F.Cu) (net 31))
 (segment (start 170.18 52.07) (end 180.34 41.91) (width 0.25) (layer B.Cu) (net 2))
 (segment (start 185.42 41.91) (end 186.69 40.64) (width 0.25) (layer B.Cu) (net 2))
 (segment (start 180.34 41.91) (end 185.42 41.91) (width 0.25) (layer B.Cu) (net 2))
 (segment (start 167.64 52.07) (end 167.64 64.77) (width 0.25) (layer B.Cu) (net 33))
 (segment (start 167.64 64.77) (end 171.45 68.58) (width 0.25) (layer B.Cu) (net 33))
 (segment (start 162.56 60.564998) (end 163.83 61.834998) (width 0.25) (layer F.Cu) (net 22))
 (segment (start 162.56 48.26) (end 162.56 60.564998) (width 0.25) (layer F.Cu) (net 22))
 (segment (start 163.83 73.66) (end 165.91999 75.74999) (width 0.25) (layer F.Cu) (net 22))
 (segment (start 163.83 61.834998) (end 163.83 73.66) (width 0.25) (layer F.Cu) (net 22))
 (segment (start 165.91999 75.74999) (end 202.38001 75.74999) (width 0.25) (layer F.Cu) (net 22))
 (segment (start 204.47 73.66) (end 204.47 68.58) (width 0.25) (layer F.Cu) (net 22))
 (segment (start 202.38001 75.74999) (end 204.47 73.66) (width 0.25) (layer F.Cu) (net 22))
 (segment (start 223.52 60.96) (end 223.52 64.77) (width 0.25) (layer B.Cu) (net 16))
 (segment (start 223.52 64.77) (end 222.25 66.04) (width 0.25) (layer B.Cu) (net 16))
 (segment (start 222.25 66.04) (end 213.36 66.04) (width 0.25) (layer B.Cu) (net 16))
 (segment (start 212.09 67.31) (end 212.09 68.58) (width 0.25) (layer B.Cu) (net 16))
 (segment (start 213.36 66.04) (end 212.09 67.31) (width 0.25) (layer B.Cu) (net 16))
 (segment (start 162.56 62.23) (end 162.56 73.66) (width 0.25) (layer F.Cu) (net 20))
 (segment (start 162.56 73.66) (end 165.1 76.2) (width 0.25) (layer F.Cu) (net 20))
 (segment (start 165.1 76.2) (end 203.2 76.2) (width 0.25) (layer F.Cu) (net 20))
 (segment (start 207.01 72.39) (end 207.01 68.58) (width 0.25) (layer F.Cu) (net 20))
 (segment (start 203.2 76.2) (end 207.01 72.39) (width 0.25) (layer F.Cu) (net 20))
 (segment (start 224.645001 61.500001) (end 220.105002 66.04) (width 0.25) (layer F.Cu) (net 18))
 (segment (start 224.645001 49.385001) (end 224.645001 61.500001) (width 0.25) (layer F.Cu) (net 18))
 (segment (start 223.52 48.26) (end 224.645001 49.385001) (width 0.25) (layer F.Cu) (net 18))
 (segment (start 220.105002 66.04) (end 210.82 66.04) (width 0.25) (layer F.Cu) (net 18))
 (segment (start 209.55 67.31) (end 209.55 68.58) (width 0.25) (layer F.Cu) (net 18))
 (segment (start 210.82 66.04) (end 209.55 67.31) (width 0.25) (layer F.Cu) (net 18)))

